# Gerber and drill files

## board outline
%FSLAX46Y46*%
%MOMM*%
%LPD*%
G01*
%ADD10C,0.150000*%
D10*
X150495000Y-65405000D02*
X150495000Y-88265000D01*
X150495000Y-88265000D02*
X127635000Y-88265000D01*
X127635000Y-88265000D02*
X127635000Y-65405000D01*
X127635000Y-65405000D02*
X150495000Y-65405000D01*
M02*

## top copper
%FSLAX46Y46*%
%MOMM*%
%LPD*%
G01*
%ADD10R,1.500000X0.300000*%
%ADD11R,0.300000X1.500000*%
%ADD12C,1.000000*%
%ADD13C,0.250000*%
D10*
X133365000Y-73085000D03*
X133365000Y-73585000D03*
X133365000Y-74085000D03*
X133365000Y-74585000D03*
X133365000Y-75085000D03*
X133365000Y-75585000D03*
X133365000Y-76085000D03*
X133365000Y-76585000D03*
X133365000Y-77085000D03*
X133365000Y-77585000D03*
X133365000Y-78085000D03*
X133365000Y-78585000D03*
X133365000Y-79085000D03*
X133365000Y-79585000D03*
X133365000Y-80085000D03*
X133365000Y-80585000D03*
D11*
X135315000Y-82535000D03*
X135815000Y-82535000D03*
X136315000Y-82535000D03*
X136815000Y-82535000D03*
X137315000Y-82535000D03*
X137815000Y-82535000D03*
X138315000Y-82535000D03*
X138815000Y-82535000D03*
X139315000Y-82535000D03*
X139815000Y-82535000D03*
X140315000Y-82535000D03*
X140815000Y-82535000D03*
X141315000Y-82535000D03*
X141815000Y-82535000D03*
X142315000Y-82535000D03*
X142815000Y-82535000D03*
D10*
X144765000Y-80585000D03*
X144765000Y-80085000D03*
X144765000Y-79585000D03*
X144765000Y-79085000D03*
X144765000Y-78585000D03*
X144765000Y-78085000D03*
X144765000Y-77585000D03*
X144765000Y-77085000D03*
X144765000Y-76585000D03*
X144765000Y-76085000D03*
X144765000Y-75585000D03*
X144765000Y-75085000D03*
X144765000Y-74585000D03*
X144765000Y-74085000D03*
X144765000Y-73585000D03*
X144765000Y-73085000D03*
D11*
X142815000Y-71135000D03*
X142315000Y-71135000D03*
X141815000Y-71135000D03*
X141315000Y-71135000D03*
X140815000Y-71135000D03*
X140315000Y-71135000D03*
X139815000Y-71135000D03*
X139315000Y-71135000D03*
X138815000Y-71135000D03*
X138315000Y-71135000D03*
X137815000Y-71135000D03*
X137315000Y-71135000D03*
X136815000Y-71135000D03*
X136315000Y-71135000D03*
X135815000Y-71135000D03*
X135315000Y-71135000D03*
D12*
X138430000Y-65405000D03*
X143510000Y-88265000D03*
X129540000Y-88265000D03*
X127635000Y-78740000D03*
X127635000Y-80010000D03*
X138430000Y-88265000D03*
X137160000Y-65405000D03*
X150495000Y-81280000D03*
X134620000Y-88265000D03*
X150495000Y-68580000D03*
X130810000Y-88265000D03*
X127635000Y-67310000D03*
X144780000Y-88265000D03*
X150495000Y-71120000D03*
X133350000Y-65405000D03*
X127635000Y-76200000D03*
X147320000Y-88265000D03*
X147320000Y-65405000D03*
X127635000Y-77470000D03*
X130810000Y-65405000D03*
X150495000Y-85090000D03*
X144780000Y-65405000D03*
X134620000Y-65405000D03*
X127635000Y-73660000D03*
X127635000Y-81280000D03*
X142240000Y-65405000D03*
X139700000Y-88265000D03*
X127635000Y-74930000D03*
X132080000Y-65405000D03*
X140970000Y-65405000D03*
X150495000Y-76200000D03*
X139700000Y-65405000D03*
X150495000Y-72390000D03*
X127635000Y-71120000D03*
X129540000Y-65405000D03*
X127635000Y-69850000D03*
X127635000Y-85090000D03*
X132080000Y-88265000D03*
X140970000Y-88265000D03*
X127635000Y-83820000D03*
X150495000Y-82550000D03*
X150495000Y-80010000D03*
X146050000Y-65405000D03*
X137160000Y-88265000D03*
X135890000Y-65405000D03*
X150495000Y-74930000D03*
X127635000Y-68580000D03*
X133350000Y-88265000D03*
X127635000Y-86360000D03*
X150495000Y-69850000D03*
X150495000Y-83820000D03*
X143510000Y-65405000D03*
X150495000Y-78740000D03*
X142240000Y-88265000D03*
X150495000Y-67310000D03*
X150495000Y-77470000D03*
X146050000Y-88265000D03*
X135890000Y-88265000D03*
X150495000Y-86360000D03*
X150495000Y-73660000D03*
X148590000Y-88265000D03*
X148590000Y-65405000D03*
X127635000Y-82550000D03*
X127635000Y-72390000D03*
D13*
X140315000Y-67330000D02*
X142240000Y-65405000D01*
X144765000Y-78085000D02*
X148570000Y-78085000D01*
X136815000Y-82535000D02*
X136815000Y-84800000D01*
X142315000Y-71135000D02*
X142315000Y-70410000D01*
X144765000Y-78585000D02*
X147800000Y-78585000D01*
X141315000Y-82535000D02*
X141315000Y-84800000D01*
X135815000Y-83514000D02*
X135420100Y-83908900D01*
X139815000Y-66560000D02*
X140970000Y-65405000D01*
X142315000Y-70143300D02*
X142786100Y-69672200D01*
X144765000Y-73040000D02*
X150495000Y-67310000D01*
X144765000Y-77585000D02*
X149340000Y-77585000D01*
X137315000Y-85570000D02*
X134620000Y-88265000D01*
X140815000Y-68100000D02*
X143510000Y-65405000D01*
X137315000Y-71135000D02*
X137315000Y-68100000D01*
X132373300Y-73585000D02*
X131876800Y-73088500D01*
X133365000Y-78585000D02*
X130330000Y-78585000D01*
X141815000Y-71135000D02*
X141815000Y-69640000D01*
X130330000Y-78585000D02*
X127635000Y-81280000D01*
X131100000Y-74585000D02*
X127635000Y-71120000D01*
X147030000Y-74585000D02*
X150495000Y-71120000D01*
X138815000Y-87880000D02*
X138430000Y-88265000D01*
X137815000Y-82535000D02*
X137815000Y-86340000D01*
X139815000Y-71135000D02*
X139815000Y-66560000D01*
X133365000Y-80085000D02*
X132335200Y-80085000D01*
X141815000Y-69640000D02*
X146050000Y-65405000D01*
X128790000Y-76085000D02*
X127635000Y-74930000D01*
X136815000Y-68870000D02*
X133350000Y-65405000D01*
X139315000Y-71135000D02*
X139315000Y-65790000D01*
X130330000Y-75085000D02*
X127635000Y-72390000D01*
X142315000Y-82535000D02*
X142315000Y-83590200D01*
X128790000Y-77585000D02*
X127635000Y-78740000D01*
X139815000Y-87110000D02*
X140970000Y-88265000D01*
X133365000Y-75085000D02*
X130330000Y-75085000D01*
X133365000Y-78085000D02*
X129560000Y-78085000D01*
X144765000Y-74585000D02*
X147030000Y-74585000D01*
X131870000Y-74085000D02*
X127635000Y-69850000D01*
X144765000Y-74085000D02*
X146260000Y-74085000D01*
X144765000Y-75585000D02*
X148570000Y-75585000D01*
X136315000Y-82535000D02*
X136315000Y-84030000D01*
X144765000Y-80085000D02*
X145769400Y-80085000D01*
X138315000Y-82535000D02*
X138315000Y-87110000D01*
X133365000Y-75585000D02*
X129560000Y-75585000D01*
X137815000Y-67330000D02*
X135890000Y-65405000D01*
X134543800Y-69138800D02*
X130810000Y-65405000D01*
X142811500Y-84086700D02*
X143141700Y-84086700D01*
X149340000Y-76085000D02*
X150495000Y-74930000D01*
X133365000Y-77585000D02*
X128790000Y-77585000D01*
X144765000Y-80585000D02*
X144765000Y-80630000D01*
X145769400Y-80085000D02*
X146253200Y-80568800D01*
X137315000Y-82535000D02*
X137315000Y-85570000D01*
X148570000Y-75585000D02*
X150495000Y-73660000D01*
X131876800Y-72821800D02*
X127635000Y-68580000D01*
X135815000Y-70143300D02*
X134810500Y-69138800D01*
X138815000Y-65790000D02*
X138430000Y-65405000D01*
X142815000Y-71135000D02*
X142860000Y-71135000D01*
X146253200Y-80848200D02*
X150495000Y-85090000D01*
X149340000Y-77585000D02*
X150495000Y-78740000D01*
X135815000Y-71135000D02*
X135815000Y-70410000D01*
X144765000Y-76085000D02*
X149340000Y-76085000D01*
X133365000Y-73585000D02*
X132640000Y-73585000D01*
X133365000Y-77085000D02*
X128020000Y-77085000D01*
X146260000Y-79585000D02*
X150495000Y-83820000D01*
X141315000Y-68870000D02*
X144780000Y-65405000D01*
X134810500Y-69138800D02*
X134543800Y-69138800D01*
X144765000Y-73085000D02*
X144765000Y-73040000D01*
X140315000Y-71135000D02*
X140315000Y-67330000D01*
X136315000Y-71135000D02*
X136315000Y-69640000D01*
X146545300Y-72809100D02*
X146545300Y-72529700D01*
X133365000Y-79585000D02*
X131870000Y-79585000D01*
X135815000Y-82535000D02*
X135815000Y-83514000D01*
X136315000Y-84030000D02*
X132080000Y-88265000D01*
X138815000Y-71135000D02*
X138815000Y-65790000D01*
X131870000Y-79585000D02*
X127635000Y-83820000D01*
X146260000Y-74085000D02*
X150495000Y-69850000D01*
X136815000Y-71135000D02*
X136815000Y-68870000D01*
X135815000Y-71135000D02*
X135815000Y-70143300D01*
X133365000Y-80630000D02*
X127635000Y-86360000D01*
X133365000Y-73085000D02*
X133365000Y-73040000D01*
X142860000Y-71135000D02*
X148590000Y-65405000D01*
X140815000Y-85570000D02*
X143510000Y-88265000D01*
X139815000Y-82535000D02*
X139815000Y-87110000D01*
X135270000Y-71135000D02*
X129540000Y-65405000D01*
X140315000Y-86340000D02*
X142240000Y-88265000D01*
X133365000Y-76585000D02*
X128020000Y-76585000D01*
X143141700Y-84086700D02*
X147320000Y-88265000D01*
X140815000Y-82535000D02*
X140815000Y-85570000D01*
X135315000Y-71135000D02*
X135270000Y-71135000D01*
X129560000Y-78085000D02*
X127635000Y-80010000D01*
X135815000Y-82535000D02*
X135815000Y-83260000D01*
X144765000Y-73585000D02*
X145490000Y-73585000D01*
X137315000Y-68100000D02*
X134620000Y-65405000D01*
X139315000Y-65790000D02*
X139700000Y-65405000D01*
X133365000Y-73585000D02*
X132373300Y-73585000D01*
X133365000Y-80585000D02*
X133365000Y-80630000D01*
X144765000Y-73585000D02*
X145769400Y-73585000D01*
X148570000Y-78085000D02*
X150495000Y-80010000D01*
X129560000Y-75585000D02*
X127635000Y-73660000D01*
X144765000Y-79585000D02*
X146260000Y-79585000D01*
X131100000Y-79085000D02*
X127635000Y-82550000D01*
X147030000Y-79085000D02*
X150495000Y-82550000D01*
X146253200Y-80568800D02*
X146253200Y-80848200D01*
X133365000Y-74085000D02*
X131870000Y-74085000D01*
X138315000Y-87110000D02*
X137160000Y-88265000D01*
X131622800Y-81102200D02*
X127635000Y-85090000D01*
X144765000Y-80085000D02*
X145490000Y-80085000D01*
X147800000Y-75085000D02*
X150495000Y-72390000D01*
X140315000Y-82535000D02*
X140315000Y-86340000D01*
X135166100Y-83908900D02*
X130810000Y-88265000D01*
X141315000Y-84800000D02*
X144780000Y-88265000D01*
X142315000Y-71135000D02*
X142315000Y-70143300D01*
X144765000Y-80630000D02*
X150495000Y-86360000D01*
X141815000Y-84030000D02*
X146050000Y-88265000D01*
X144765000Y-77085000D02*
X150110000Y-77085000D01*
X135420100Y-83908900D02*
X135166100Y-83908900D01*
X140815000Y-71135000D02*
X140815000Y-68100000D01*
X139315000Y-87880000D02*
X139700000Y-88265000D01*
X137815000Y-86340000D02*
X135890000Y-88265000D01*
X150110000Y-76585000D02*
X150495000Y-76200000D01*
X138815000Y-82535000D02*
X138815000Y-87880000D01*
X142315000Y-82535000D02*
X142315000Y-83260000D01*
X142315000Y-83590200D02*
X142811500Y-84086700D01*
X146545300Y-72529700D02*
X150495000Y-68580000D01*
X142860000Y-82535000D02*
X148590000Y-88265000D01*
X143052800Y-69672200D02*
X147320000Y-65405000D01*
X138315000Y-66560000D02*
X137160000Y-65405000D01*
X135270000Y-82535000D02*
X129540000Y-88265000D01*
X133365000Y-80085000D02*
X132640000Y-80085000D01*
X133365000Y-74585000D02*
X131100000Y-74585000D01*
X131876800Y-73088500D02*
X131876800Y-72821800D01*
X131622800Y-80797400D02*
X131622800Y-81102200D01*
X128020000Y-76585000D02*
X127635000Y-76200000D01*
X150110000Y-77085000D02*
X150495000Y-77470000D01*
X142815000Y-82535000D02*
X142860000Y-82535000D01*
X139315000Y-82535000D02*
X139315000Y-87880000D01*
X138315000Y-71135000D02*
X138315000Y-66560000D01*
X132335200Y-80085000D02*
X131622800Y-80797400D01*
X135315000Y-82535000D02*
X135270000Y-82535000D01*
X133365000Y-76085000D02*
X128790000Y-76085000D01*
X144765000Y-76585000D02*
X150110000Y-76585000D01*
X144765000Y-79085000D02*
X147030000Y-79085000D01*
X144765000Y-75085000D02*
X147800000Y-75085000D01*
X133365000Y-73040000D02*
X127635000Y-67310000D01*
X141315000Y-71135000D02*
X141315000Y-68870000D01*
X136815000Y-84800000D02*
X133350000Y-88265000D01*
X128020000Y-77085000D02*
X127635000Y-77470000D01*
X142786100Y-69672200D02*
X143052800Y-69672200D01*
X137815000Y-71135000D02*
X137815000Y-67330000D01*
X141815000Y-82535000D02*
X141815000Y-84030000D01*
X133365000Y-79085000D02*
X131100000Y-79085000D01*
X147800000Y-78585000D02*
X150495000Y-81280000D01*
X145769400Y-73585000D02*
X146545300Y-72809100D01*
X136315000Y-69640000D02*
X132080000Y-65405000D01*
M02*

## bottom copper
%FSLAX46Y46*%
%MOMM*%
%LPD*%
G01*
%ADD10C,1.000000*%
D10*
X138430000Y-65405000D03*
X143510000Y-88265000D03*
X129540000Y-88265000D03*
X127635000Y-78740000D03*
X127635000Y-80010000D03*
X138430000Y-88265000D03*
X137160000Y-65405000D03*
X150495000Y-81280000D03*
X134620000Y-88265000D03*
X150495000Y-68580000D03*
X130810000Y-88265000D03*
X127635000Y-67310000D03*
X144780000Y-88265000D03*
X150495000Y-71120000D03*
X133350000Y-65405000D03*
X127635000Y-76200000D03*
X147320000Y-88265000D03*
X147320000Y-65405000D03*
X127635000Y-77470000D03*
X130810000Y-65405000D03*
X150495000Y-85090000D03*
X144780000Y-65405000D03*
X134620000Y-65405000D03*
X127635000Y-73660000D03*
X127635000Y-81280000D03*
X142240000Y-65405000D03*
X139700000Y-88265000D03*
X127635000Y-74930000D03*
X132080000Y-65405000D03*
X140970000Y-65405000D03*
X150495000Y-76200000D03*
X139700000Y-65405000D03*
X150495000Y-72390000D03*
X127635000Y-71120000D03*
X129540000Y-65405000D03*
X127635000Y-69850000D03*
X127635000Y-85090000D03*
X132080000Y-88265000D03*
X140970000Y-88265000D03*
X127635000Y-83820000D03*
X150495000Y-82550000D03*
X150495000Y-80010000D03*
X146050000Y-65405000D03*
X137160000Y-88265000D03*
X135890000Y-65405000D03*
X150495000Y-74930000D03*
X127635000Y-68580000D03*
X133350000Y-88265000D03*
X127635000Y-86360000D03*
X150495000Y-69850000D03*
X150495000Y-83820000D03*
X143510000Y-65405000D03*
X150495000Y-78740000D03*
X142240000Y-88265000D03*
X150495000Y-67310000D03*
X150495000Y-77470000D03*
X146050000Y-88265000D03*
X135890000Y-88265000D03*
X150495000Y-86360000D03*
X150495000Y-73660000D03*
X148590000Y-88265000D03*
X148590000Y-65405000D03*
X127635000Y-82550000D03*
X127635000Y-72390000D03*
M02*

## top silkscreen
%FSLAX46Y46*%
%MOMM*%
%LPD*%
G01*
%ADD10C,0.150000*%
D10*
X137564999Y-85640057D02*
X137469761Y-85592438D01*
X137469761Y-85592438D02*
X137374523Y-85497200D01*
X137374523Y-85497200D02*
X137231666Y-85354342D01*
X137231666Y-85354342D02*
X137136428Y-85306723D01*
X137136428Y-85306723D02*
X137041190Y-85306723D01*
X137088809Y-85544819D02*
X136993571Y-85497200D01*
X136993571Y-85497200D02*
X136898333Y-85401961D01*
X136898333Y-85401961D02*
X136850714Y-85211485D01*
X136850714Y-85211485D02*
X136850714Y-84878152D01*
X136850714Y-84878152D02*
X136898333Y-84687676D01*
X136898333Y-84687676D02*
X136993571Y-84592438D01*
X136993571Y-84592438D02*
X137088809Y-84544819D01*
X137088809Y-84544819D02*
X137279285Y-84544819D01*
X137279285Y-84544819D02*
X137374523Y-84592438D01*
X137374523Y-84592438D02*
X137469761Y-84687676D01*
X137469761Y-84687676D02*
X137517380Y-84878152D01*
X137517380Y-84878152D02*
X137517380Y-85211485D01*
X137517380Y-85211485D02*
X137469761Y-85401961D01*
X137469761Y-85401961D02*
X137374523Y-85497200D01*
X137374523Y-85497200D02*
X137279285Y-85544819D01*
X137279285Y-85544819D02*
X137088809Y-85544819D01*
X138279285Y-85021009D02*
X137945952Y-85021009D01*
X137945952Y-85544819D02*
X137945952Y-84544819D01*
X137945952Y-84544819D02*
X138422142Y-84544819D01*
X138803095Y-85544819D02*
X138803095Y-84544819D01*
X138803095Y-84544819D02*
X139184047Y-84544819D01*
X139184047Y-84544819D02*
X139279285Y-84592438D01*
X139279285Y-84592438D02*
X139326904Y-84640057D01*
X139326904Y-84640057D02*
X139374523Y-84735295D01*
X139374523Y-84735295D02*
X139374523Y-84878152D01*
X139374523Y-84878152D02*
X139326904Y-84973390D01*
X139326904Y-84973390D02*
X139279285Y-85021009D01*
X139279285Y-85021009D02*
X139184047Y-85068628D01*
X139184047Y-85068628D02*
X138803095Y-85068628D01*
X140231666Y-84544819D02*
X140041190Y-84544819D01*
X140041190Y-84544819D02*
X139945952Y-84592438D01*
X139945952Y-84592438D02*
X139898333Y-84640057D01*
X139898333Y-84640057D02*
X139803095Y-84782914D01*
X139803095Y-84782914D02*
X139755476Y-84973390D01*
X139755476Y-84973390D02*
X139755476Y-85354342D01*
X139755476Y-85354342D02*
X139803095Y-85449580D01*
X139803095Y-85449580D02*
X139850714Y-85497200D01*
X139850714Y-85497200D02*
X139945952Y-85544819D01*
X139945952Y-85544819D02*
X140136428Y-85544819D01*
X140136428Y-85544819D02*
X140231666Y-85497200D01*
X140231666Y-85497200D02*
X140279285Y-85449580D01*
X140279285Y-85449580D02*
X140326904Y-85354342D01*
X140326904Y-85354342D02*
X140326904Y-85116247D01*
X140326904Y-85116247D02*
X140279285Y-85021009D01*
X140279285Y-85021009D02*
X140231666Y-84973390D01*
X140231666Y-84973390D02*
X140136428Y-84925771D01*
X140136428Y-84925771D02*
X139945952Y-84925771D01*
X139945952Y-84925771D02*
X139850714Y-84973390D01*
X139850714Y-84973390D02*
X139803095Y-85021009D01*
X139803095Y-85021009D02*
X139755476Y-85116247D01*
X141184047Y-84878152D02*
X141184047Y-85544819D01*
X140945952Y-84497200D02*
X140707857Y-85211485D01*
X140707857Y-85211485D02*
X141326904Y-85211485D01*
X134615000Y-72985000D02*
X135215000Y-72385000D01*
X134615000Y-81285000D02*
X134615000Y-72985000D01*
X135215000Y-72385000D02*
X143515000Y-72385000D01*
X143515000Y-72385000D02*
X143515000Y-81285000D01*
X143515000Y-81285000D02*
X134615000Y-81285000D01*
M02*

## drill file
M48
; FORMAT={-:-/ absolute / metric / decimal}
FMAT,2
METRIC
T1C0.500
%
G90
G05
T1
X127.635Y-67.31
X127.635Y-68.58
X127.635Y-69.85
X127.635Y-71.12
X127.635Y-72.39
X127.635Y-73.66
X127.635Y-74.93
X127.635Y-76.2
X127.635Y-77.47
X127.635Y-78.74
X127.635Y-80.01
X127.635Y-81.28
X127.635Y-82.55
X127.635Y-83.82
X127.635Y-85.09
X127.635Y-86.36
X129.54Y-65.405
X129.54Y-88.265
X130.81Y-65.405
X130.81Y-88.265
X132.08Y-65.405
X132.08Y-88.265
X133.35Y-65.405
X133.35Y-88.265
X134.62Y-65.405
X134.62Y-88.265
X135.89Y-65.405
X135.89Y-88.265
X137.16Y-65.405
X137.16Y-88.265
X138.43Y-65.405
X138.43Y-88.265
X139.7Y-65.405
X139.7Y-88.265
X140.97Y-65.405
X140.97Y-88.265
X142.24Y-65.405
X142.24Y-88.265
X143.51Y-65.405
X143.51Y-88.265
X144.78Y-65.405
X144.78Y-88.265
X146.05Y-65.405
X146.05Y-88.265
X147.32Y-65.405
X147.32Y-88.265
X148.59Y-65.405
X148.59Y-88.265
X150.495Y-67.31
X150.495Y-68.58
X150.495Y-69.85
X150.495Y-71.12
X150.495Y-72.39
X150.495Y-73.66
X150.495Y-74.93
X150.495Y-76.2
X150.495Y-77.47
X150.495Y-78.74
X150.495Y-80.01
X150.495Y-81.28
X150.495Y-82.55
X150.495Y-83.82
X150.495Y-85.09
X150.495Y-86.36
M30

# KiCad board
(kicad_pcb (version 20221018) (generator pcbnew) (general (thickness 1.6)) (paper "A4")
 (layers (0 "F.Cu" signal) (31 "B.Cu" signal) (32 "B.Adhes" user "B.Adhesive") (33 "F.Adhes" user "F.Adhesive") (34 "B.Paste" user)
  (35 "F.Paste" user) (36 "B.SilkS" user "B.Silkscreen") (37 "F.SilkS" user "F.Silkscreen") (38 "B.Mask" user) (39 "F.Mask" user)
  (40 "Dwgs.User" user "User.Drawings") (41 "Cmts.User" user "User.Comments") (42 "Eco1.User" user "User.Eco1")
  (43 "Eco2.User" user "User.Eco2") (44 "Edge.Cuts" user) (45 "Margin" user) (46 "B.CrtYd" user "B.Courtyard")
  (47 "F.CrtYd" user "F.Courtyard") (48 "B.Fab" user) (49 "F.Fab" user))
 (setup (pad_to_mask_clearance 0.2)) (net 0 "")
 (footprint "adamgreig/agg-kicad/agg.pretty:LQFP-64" (layer "F.Cu") (at 139.065 76.835)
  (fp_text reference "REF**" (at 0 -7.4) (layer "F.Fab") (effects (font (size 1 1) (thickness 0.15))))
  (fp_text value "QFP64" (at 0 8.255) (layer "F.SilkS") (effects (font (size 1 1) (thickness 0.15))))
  (fp_line (start -4.45 -3.85) (end -3.85 -4.45) (stroke (width 0.15) (type solid)) (layer "F.SilkS"))
  (fp_line (start -4.45 4.45) (end -4.45 -3.85) (stroke (width 0.15) (type solid)) (layer "F.SilkS"))
  (fp_line (start -3.85 -4.45) (end 4.45 -4.45) (stroke (width 0.15) (type solid)) (layer "F.SilkS"))
  (fp_line (start 4.45 -4.45) (end 4.45 4.45) (stroke (width 0.15) (type solid)) (layer "F.SilkS"))
  (fp_line (start 4.45 4.45) (end -4.45 4.45) (stroke (width 0.15) (type solid)) (layer "F.SilkS"))
  (pad "1" smd rect (at -5.7 -3.75) (size 1.5 0.3) (layers "F.Cu" "F.Paste" "F.Mask"))
  (pad "2" smd rect (at -5.7 -3.25) (size 1.5 0.3) (layers "F.Cu" "F.Paste" "F.Mask"))
  (pad "3" smd rect (at -5.7 -2.75) (size 1.5 0.3) (layers "F.Cu" "F.Paste" "F.Mask"))
  (pad "4" smd rect (at -5.7 -2.25) (size 1.5 0.3) (layers "F.Cu" "F.Paste" "F.Mask"))
  (pad "5" smd rect (at -5.7 -1.75) (size 1.5 0.3) (layers "F.Cu" "F.Paste" "F.Mask"))
  (pad "6" smd rect (at -5.7 -1.25) (size 1.5 0.3) (layers "F.Cu" "F.Paste" "F.Mask"))
  (pad "7" smd rect (at -5.7 -0.75) (size 1.5 0.3) (layers "F.Cu" "F.Paste" "F.Mask"))
  (pad "8" smd rect (at -5.7 -0.25) (size 1.5 0.3) (layers "F.Cu" "F.Paste" "F.Mask"))
  (pad "9" smd rect (at -5.7 0.25) (size 1.5 0.3) (layers "F.Cu" "F.Paste" "F.Mask"))
  (pad "10" smd rect (at -5.7 0.75) (size 1.5 0.3) (layers "F.Cu" "F.Paste" "F.Mask"))
  (pad "11" smd rect (at -5.7 1.25) (size 1.5 0.3) (layers "F.Cu" "F.Paste" "F.Mask"))
  (pad "12" smd rect (at -5.7 1.75) (size 1.5 0.3) (layers "F.Cu" "F.Paste" "F.Mask"))
  (pad "13" smd rect (at -5.7 2.25) (size 1.5 0.3) (layers "F.Cu" "F.Paste" "F.Mask"))
  (pad "14" smd rect (at -5.7 2.75) (size 1.5 0.3) (layers "F.Cu" "F.Paste" "F.Mask"))
  (pad "15" smd rect (at -5.7 3.25) (size 1.5 0.3) (layers "F.Cu" "F.Paste" "F.Mask"))
  (pad "16" smd rect (at -5.7 3.75) (size 1.5 0.3) (layers "F.Cu" "F.Paste" "F.Mask"))
  (pad "17" smd rect (at -3.75 5.7) (size 0.3 1.5) (layers "F.Cu" "F.Paste" "F.Mask"))
  (pad "18" smd rect (at -3.25 5.7) (size 0.3 1.5) (layers "F.Cu" "F.Paste" "F.Mask"))
  (pad "19" smd rect (at -2.75 5.7) (size 0.3 1.5) (layers "F.Cu" "F.Paste" "F.Mask"))
  (pad "20" smd rect (at -2.25 5.7) (size 0.3 1.5) (layers "F.Cu" "F.Paste" "F.Mask"))
  (pad "21" smd rect (at -1.75 5.7) (size 0.3 1.5) (layers "F.Cu" "F.Paste" "F.Mask"))
  (pad "22" smd rect (at -1.25 5.7) (size 0.3 1.5) (layers "F.Cu" "F.Paste" "F.Mask"))
  (pad "23" smd rect (at -0.75 5.7) (size 0.3 1.5) (layers "F.Cu" "F.Paste" "F.Mask"))
  (pad "24" smd rect (at -0.25 5.7) (size 0.3 1.5) (layers "F.Cu" "F.Paste" "F.Mask"))
  (pad "25" smd rect (at 0.25 5.7) (size 0.3 1.5) (layers "F.Cu" "F.Paste" "F.Mask"))
  (pad "26" smd rect (at 0.75 5.7) (size 0.3 1.5) (layers "F.Cu" "F.Paste" "F.Mask"))
  (pad "27" smd rect (at 1.25 5.7) (size 0.3 1.5) (layers "F.Cu" "F.Paste" "F.Mask"))
  (pad "28" smd rect (at 1.75 5.7) (size 0.3 1.5) (layers "F.Cu" "F.Paste" "F.Mask"))
  (pad "29" smd rect (at 2.25 5.7) (size 0.3 1.5) (layers "F.Cu" "F.Paste" "F.Mask"))
  (pad "30" smd rect (at 2.75 5.7) (size 0.3 1.5) (layers "F.Cu" "F.Paste" "F.Mask"))
  (pad "31" smd rect (at 3.25 5.7) (size 0.3 1.5) (layers "F.Cu" "F.Paste" "F.Mask"))
  (pad "32" smd rect (at 3.75 5.7) (size 0.3 1.5) (layers "F.Cu" "F.Paste" "F.Mask"))
  (pad "33" smd rect (at 5.7 3.75) (size 1.5 0.3) (layers "F.Cu" "F.Paste" "F.Mask"))
  (pad "34" smd rect (at 5.7 3.25) (size 1.5 0.3) (layers "F.Cu" "F.Paste" "F.Mask"))
  (pad "35" smd rect (at 5.7 2.75) (size 1.5 0.3) (layers "F.Cu" "F.Paste" "F.Mask"))
  (pad "36" smd rect (at 5.7 2.25) (size 1.5 0.3) (layers "F.Cu" "F.Paste" "F.Mask"))
  (pad "37" smd rect (at 5.7 1.75) (size 1.5 0.3) (layers "F.Cu" "F.Paste" "F.Mask"))
  (pad "38" smd rect (at 5.7 1.25) (size 1.5 0.3) (layers "F.Cu" "F.Paste" "F.Mask"))
  (pad "39" smd rect (at 5.7 0.75) (size 1.5 0.3) (layers "F.Cu" "F.Paste" "F.Mask"))
  (pad "40" smd rect (at 5.7 0.25) (size 1.5 0.3) (layers "F.Cu" "F.Paste" "F.Mask"))
  (pad "41" smd rect (at 5.7 -0.25) (size 1.5 0.3) (layers "F.Cu" "F.Paste" "F.Mask"))
  (pad "42" smd rect (at 5.7 -0.75) (size 1.5 0.3) (layers "F.Cu" "F.Paste" "F.Mask"))
  (pad "43" smd rect (at 5.7 -1.25) (size 1.5 0.3) (layers "F.Cu" "F.Paste" "F.Mask"))
  (pad "44" smd rect (at 5.7 -1.75) (size 1.5 0.3) (layers "F.Cu" "F.Paste" "F.Mask"))
  (pad "45" smd rect (at 5.7 -2.25) (size 1.5 0.3) (layers "F.Cu" "F.Paste" "F.Mask"))
  (pad "46" smd rect (at 5.7 -2.75) (size 1.5 0.3) (layers "F.Cu" "F.Paste" "F.Mask"))
  (pad "47" smd rect (at 5.7 -3.25) (size 1.5 0.3) (layers "F.Cu" "F.Paste" "F.Mask"))
  (pad "48" smd rect (at 5.7 -3.75) (size 1.5 0.3) (layers "F.Cu" "F.Paste" "F.Mask"))
  (pad "49" smd rect (at 3.75 -5.7) (size 0.3 1.5) (layers "F.Cu" "F.Paste" "F.Mask"))
  (pad "50" smd rect (at 3.25 -5.7) (size 0.3 1.5) (layers "F.Cu" "F.Paste" "F.Mask"))
  (pad "51" smd rect (at 2.75 -5.7) (size 0.3 1.5) (layers "F.Cu" "F.Paste" "F.Mask"))
  (pad "52" smd rect (at 2.25 -5.7) (size 0.3 1.5) (layers "F.Cu" "F.Paste" "F.Mask"))
  (pad "53" smd rect (at 1.75 -5.7) (size 0.3 1.5) (layers "F.Cu" "F.Paste" "F.Mask"))
  (pad "54" smd rect (at 1.25 -5.7) (size 0.3 1.5) (layers "F.Cu" "F.Paste" "F.Mask"))
  (pad "55" smd rect (at 0.75 -5.7) (size 0.3 1.5) (layers "F.Cu" "F.Paste" "F.Mask"))
  (pad "56" smd rect (at 0.25 -5.7) (size 0.3 1.5) (layers "F.Cu" "F.Paste" "F.Mask"))
  (pad "57" smd rect (at -0.25 -5.7) (size 0.3 1.5) (layers "F.Cu" "F.Paste" "F.Mask"))
  (pad "58" smd rect (at -0.75 -5.7) (size 0.3 1.5) (layers "F.Cu" "F.Paste" "F.Mask"))
  (pad "59" smd rect (at -1.25 -5.7) (size 0.3 1.5) (layers "F.Cu" "F.Paste" "F.Mask"))
  (pad "60" smd rect (at -1.75 -5.7) (size 0.3 1.5) (layers "F.Cu" "F.Paste" "F.Mask"))
  (pad "61" smd rect (at -2.25 -5.7) (size 0.3 1.5) (layers "F.Cu" "F.Paste" "F.Mask"))
  (pad "62" smd rect (at -2.75 -5.7) (size 0.3 1.5) (layers "F.Cu" "F.Paste" "F.Mask"))
  (pad "63" smd rect (at -3.25 -5.7) (size 0.3 1.5) (layers "F.Cu" "F.Paste" "F.Mask"))
  (pad "64" smd rect (at -3.75 -5.7) (size 0.3 1.5) (layers "F.Cu" "F.Paste" "F.Mask")))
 (gr_line (start 150.495 65.405) (end 150.495 88.265) (stroke (width 0.15) (type solid)) (layer "Edge.Cuts"))
 (gr_line (start 150.495 88.265) (end 127.635 88.265) (stroke (width 0.15) (type solid)) (layer "Edge.Cuts"))
 (gr_line (start 127.635 88.265) (end 127.635 65.405) (stroke (width 0.15) (type solid)) (layer "Edge.Cuts"))
 (gr_line (start 127.635 65.405) (end 150.495 65.405) (stroke (width 0.15) (type solid)) (layer "Edge.Cuts"))
 (segment (start 140.315 67.33) (end 142.24 65.405) (width 0.25) (layer "F.Cu") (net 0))
 (segment (start 144.765 78.085) (end 148.57 78.085) (width 0.25) (layer "F.Cu") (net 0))
 (segment (start 136.815 82.535) (end 136.815 84.8) (width 0.25) (layer "F.Cu") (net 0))
 (segment (start 142.315 71.135) (end 142.315 70.41) (width 0.25) (layer "F.Cu") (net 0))
 (segment (start 144.765 78.585) (end 147.8 78.585) (width 0.25) (layer "F.Cu") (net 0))
 (segment (start 141.315 82.535) (end 141.315 84.8) (width 0.25) (layer "F.Cu") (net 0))
 (segment (start 135.815 83.514) (end 135.4201 83.9089) (width 0.25) (layer "F.Cu") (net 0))
 (segment (start 139.815 66.56) (end 140.97 65.405) (width 0.25) (layer "F.Cu") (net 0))
 (segment (start 142.315 70.1433) (end 142.7861 69.6722) (width 0.25) (layer "F.Cu") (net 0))
 (segment (start 144.765 73.04) (end 150.495 67.31) (width 0.25) (layer "F.Cu") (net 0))
 (segment (start 144.765 77.585) (end 149.34 77.585) (width 0.25) (layer "F.Cu") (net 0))
 (segment (start 137.315 85.57) (end 134.62 88.265) (width 0.25) (layer "F.Cu") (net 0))
 (segment (start 140.815 68.1) (end 143.51 65.405) (width 0.25) (layer "F.Cu") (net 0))
 (segment (start 137.315 71.135) (end 137.315 68.1) (width 0.25) (layer "F.Cu") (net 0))
 (segment (start 132.3733 73.585) (end 131.8768 73.0885) (width 0.25) (layer "F.Cu") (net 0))
 (segment (start 133.365 78.585) (end 130.33 78.585) (width 0.25) (layer "F.Cu") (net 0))
 (segment (start 141.815 71.135) (end 141.815 69.64) (width 0.25) (layer "F.Cu") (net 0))
 (segment (start 130.33 78.585) (end 127.635 81.28) (width 0.25) (layer "F.Cu") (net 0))
 (segment (start 131.1 74.585) (end 127.635 71.12) (width 0.25) (layer "F.Cu") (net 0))
 (segment (start 147.03 74.585) (end 150.495 71.12) (width 0.25) (layer "F.Cu") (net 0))
 (segment (start 138.815 87.88) (end 138.43 88.265) (width 0.25) (layer "F.Cu") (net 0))
 (segment (start 137.815 82.535) (end 137.815 86.34) (width 0.25) (layer "F.Cu") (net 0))
 (segment (start 139.815 71.135) (end 139.815 66.56) (width 0.25) (layer "F.Cu") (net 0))
 (segment (start 133.365 80.085) (end 132.3352 80.085) (width 0.25) (layer "F.Cu") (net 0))
 (segment (start 141.815 69.64) (end 146.05 65.405) (width 0.25) (layer "F.Cu") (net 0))
 (segment (start 128.79 76.085) (end 127.635 74.93) (width 0.25) (layer "F.Cu") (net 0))
 (segment (start 136.815 68.87) (end 133.35 65.405) (width 0.25) (layer "F.Cu") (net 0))
 (segment (start 139.315 71.135) (end 139.315 65.79) (width 0.25) (layer "F.Cu") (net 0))
 (segment (start 130.33 75.085) (end 127.635 72.39) (width 0.25) (layer "F.Cu") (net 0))
 (segment (start 142.315 82.535) (end 142.315 83.5902) (width 0.25) (layer "F.Cu") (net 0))
 (segment (start 128.79 77.585) (end 127.635 78.74) (width 0.25) (layer "F.Cu") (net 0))
 (segment (start 139.815 87.11) (end 140.97 88.265) (width 0.25) (layer "F.Cu") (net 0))
 (segment (start 133.365 75.085) (end 130.33 75.085) (width 0.25) (layer "F.Cu") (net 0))
 (segment (start 133.365 78.085) (end 129.56 78.085) (width 0.25) (layer "F.Cu") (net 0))
 (segment (start 144.765 74.585) (end 147.03 74.585) (width 0.25) (layer "F.Cu") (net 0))
 (segment (start 131.87 74.085) (end 127.635 69.85) (width 0.25) (layer "F.Cu") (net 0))
 (segment (start 144.765 74.085) (end 146.26 74.085) (width 0.25) (layer "F.Cu") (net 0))
 (segment (start 144.765 75.585) (end 148.57 75.585) (width 0.25) (layer "F.Cu") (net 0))
 (segment (start 136.315 82.535) (end 136.315 84.03) (width 0.25) (layer "F.Cu") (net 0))
 (segment (start 144.765 80.085) (end 145.7694 80.085) (width 0.25) (layer "F.Cu") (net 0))
 (segment (start 138.315 82.535) (end 138.315 87.11) (width 0.25) (layer "F.Cu") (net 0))
 (segment (start 133.365 75.585) (end 129.56 75.585) (width 0.25) (layer "F.Cu") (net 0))
 (segment (start 137.815 67.33) (end 135.89 65.405) (width 0.25) (layer "F.Cu") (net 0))
 (segment (start 134.5438 69.1388) (end 130.81 65.405) (width 0.25) (layer "F.Cu") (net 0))
 (segment (start 142.8115 84.0867) (end 143.1417 84.0867) (width 0.25) (layer "F.Cu") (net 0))
 (segment (start 149.34 76.085) (end 150.495 74.93) (width 0.25) (layer "F.Cu") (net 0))
 (segment (start 133.365 77.585) (end 128.79 77.585) (width 0.25) (layer "F.Cu") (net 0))
 (segment (start 144.765 80.585) (end 144.765 80.63) (width 0.25) (layer "F.Cu") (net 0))
 (segment (start 145.7694 80.085) (end 146.2532 80.5688) (width 0.25) (layer "F.Cu") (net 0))
 (segment (start 137.315 82.535) (end 137.315 85.57) (width 0.25) (layer "F.Cu") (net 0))
 (segment (start 148.57 75.585) (end 150.495 73.66) (width 0.25) (layer "F.Cu") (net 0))
 (segment (start 131.8768 72.8218) (end 127.635 68.58) (width 0.25) (layer "F.Cu") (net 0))
 (segment (start 135.815 70.1433) (end 134.8105 69.1388) (width 0.25) (layer "F.Cu") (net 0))
 (segment (start 138.815 65.79) (end 138.43 65.405) (width 0.25) (layer "F.Cu") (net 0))
 (segment (start 142.815 71.135) (end 142.86 71.135) (width 0.25) (layer "F.Cu") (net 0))
 (segment (start 146.2532 80.8482) (end 150.495 85.09) (width 0.25) (layer "F.Cu") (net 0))
 (segment (start 149.34 77.585) (end 150.495 78.74) (width 0.25) (layer "F.Cu") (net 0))
 (segment (start 135.815 71.135) (end 135.815 70.41) (width 0.25) (layer "F.Cu") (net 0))
 (segment (start 144.765 76.085) (end 149.34 76.085) (width 0.25) (layer "F.Cu") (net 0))
 (segment (start 133.365 73.585) (end 132.64 73.585) (width 0.25) (layer "F.Cu") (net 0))
 (segment (start 133.365 77.085) (end 128.02 77.085) (width 0.25) (layer "F.Cu") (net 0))
 (segment (start 146.26 79.585) (end 150.495 83.82) (width 0.25) (layer "F.Cu") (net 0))
 (segment (start 141.315 68.87) (end 144.78 65.405) (width 0.25) (layer "F.Cu") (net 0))
 (segment (start 134.8105 69.1388) (end 134.5438 69.1388) (width 0.25) (layer "F.Cu") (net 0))
 (segment (start 144.765 73.085) (end 144.765 73.04) (width 0.25) (layer "F.Cu") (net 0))
 (segment (start 140.315 71.135) (end 140.315 67.33) (width 0.25) (layer "F.Cu") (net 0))
 (segment (start 136.315 71.135) (end 136.315 69.64) (width 0.25) (layer "F.Cu") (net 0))
 (segment (start 146.5453 72.8091) (end 146.5453 72.5297) (width 0.25) (layer "F.Cu") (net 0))
 (segment (start 133.365 79.585) (end 131.87 79.585) (width 0.25) (layer "F.Cu") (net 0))
 (segment (start 135.815 82.535) (end 135.815 83.514) (width 0.25) (layer "F.Cu") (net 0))
 (segment (start 136.315 84.03) (end 132.08 88.265) (width 0.25) (layer "F.Cu") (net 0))
 (segment (start 138.815 71.135) (end 138.815 65.79) (width 0.25) (layer "F.Cu") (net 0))
 (segment (start 131.87 79.585) (end 127.635 83.82) (width 0.25) (layer "F.Cu") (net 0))
 (segment (start 146.26 74.085) (end 150.495 69.85) (width 0.25) (layer "F.Cu") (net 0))
 (segment (start 136.815 71.135) (end 136.815 68.87) (width 0.25) (layer "F.Cu") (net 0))
 (segment (start 135.815 71.135) (end 135.815 70.1433) (width 0.25) (layer "F.Cu") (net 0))
 (segment (start 133.365 80.63) (end 127.635 86.36) (width 0.25) (layer "F.Cu") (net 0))
 (segment (start 133.365 73.085) (end 133.365 73.04) (width 0.25) (layer "F.Cu") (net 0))
 (segment (start 142.86 71.135) (end 148.59 65.405) (width 0.25) (layer "F.Cu") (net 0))
 (segment (start 140.815 85.57) (end 143.51 88.265) (width 0.25) (layer "F.Cu") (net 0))
 (segment (start 139.815 82.535) (end 139.815 87.11) (width 0.25) (layer "F.Cu") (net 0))
 (segment (start 135.27 71.135) (end 129.54 65.405) (width 0.25) (layer "F.Cu") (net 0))
 (segment (start 140.315 86.34) (end 142.24 88.265) (width 0.25) (layer "F.Cu") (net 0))
 (segment (start 133.365 76.585) (end 128.02 76.585) (width 0.25) (layer "F.Cu") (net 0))
 (segment (start 143.1417 84.0867) (end 147.32 88.265) (width 0.25) (layer "F.Cu") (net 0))
 (segment (start 140.815 82.535) (end 140.815 85.57) (width 0.25) (layer "F.Cu") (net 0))
 (segment (start 135.315 71.135) (end 135.27 71.135) (width 0.25) (layer "F.Cu") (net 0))
 (segment (start 129.56 78.085) (end 127.635 80.01) (width 0.25) (layer "F.Cu") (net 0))
 (segment (start 135.815 82.535) (end 135.815 83.26) (width 0.25) (layer "F.Cu") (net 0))
 (segment (start 144.765 73.585) (end 145.49 73.585) (width 0.25) (layer "F.Cu") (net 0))
 (segment (start 137.315 68.1) (end 134.62 65.405) (width 0.25) (layer "F.Cu") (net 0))
 (segment (start 139.315 65.79) (end 139.7 65.405) (width 0.25) (layer "F.Cu") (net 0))
 (segment (start 133.365 73.585) (end 132.3733 73.585) (width 0.25) (layer "F.Cu") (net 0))
 (segment (start 133.365 80.585) (end 133.365 80.63) (width 0.25) (layer "F.Cu") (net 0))
 (segment (start 144.765 73.585) (end 145.7694 73.585) (width 0.25) (layer "F.Cu") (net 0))
 (segment (start 148.57 78.085) (end 150.495 80.01) (width 0.25) (layer "F.Cu") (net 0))
 (segment (start 129.56 75.585) (end 127.635 73.66) (width 0.25) (layer "F.Cu") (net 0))
 (segment (start 144.765 79.585) (end 146.26 79.585) (width 0.25) (layer "F.Cu") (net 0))
 (segment (start 131.1 79.085) (end 127.635 82.55) (width 0.25) (layer "F.Cu") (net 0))
 (segment (start 147.03 79.085) (end 150.495 82.55) (width 0.25) (layer "F.Cu") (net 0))
 (segment (start 146.2532 80.5688) (end 146.2532 80.8482) (width 0.25) (layer "F.Cu") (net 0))
 (segment (start 133.365 74.085) (end 131.87 74.085) (width 0.25) (layer "F.Cu") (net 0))
 (segment (start 138.315 87.11) (end 137.16 88.265) (width 0.25) (layer "F.Cu") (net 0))
 (segment (start 131.6228 81.1022) (end 127.635 85.09) (width 0.25) (layer "F.Cu") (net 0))
 (segment (start 144.765 80.085) (end 145.49 80.085) (width 0.25) (layer "F.Cu") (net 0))
 (segment (start 147.8 75.085) (end 150.495 72.39) (width 0.25) (layer "F.Cu") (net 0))
 (segment (start 140.315 82.535) (end 140.315 86.34) (width 0.25) (layer "F.Cu") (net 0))
 (segment (start 135.1661 83.9089) (end 130.81 88.265) (width 0.25) (layer "F.Cu") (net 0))
 (segment (start 141.315 84.8) (end 144.78 88.265) (width 0.25) (layer "F.Cu") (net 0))
 (segment (start 142.315 71.135) (end 142.315 70.1433) (width 0.25) (layer "F.Cu") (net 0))
 (segment (start 144.765 80.63) (end 150.495 86.36) (width 0.25) (layer "F.Cu") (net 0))
 (segment (start 141.815 84.03) (end 146.05 88.265) (width 0.25) (layer "F.Cu") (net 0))
 (segment (start 144.765 77.085) (end 150.11 77.085) (width 0.25) (layer "F.Cu") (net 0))
 (segment (start 135.4201 83.9089) (end 135.1661 83.9089) (width 0.25) (layer "F.Cu") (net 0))
 (segment (start 140.815 71.135) (end 140.815 68.1) (width 0.25) (layer "F.Cu") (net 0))
 (segment (start 139.315 87.88) (end 139.7 88.265) (width 0.25) (layer "F.Cu") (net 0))
 (segment (start 137.815 86.34) (end 135.89 88.265) (width 0.25) (layer "F.Cu") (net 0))
 (segment (start 150.11 76.585) (end 150.495 76.2) (width 0.25) (layer "F.Cu") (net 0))
 (segment (start 138.815 82.535) (end 138.815 87.88) (width 0.25) (layer "F.Cu") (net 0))
 (segment (start 142.315 82.535) (end 142.315 83.26) (width 0.25) (layer "F.Cu") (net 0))
 (segment (start 142.315 83.5902) (end 142.8115 84.0867) (width 0.25) (layer "F.Cu") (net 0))
 (segment (start 146.5453 72.5297) (end 150.495 68.58) (width 0.25) (layer "F.Cu") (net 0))
 (segment (start 142.86 82.535) (end 148.59 88.265) (width 0.25) (layer "F.Cu") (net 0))
 (segment (start 143.0528 69.6722) (end 147.32 65.405) (width 0.25) (layer "F.Cu") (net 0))
 (segment (start 138.315 66.56) (end 137.16 65.405) (width 0.25) (layer "F.Cu") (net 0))
 (segment (start 135.27 82.535) (end 129.54 88.265) (width 0.25) (layer "F.Cu") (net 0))
 (segment (start 133.365 80.085) (end 132.64 80.085) (width 0.25) (layer "F.Cu") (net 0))
 (segment (start 133.365 74.585) (end 131.1 74.585) (width 0.25) (layer "F.Cu") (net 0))
 (segment (start 131.8768 73.0885) (end 131.8768 72.8218) (width 0.25) (layer "F.Cu") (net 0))
 (segment (start 131.6228 80.7974) (end 131.6228 81.1022) (width 0.25) (layer "F.Cu") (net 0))
 (segment (start 128.02 76.585) (end 127.635 76.2) (width 0.25) (layer "F.Cu") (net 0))
 (segment (start 150.11 77.085) (end 150.495 77.47) (width 0.25) (layer "F.Cu") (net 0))
 (segment (start 142.815 82.535) (end 142.86 82.535) (width 0.25) (layer "F.Cu") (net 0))
 (segment (start 139.315 82.535) (end 139.315 87.88) (width 0.25) (layer "F.Cu") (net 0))
 (segment (start 138.315 71.135) (end 138.315 66.56) (width 0.25) (layer "F.Cu") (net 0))
 (segment (start 132.3352 80.085) (end 131.6228 80.7974) (width 0.25) (layer "F.Cu") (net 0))
 (segment (start 135.315 82.535) (end 135.27 82.535) (width 0.25) (layer "F.Cu") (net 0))
 (segment (start 133.365 76.085) (end 128.79 76.085) (width 0.25) (layer "F.Cu") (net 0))
 (segment (start 144.765 76.585) (end 150.11 76.585) (width 0.25) (layer "F.Cu") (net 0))
 (segment (start 144.765 79.085) (end 147.03 79.085) (width 0.25) (layer "F.Cu") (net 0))
 (segment (start 144.765 75.085) (end 147.8 75.085) (width 0.25) (layer "F.Cu") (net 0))
 (segment (start 133.365 73.04) (end 127.635 67.31) (width 0.25) (layer "F.Cu") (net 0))
 (segment (start 141.315 71.135) (end 141.315 68.87) (width 0.25) (layer "F.Cu") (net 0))
 (segment (start 136.815 84.8) (end 133.35 88.265) (width 0.25) (layer "F.Cu") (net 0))
 (segment (start 128.02 77.085) (end 127.635 77.47) (width 0.25) (layer "F.Cu") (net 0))
 (segment (start 142.7861 69.6722) (end 143.0528 69.6722) (width 0.25) (layer "F.Cu") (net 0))
 (segment (start 137.815 71.135) (end 137.815 67.33) (width 0.25) (layer "F.Cu") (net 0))
 (segment (start 141.815 82.535) (end 141.815 84.03) (width 0.25) (layer "F.Cu") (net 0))
 (segment (start 133.365 79.085) (end 131.1 79.085) (width 0.25) (layer "F.Cu") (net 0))
 (segment (start 147.8 78.585) (end 150.495 81.28) (width 0.25) (layer "F.Cu") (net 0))
 (segment (start 145.7694 73.585) (end 146.5453 72.8091) (width 0.25) (layer "F.Cu") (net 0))
 (segment (start 136.315 69.64) (end 132.08 65.405) (width 0.25) (layer "F.Cu") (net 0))
 (via (at 138.43 65.405) (size 1) (drill 0.5) (layers "F.Cu" "B.Cu") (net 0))
 (via (at 143.51 88.265) (size 1) (drill 0.5) (layers "F.Cu" "B.Cu") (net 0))
 (via (at 129.54 88.265) (size 1) (drill 0.5) (layers "F.Cu" "B.Cu") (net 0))
 (via (at 127.635 78.74) (size 1) (drill 0.5) (layers "F.Cu" "B.Cu") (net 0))
 (via (at 127.635 80.01) (size 1) (drill 0.5) (layers "F.Cu" "B.Cu") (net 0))
 (via (at 138.43 88.265) (size 1) (drill 0.5) (layers "F.Cu" "B.Cu") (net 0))
 (via (at 137.16 65.405) (size 1) (drill 0.5) (layers "F.Cu" "B.Cu") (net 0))
 (via (at 150.495 81.28) (size 1) (drill 0.5) (layers "F.Cu" "B.Cu") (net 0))
 (via (at 134.62 88.265) (size 1) (drill 0.5) (layers "F.Cu" "B.Cu") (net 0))
 (via (at 150.495 68.58) (size 1) (drill 0.5) (layers "F.Cu" "B.Cu") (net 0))
 (via (at 130.81 88.265) (size 1) (drill 0.5) (layers "F.Cu" "B.Cu") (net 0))
 (via (at 127.635 67.31) (size 1) (drill 0.5) (layers "F.Cu" "B.Cu") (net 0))
 (via (at 144.78 88.265) (size 1) (drill 0.5) (layers "F.Cu" "B.Cu") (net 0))
 (via (at 150.495 71.12) (size 1) (drill 0.5) (layers "F.Cu" "B.Cu") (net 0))
 (via (at 133.35 65.405) (size 1) (drill 0.5) (layers "F.Cu" "B.Cu") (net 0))
 (via (at 127.635 76.2) (size 1) (drill 0.5) (layers "F.Cu" "B.Cu") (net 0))
 (via (at 147.32 88.265) (size 1) (drill 0.5) (layers "F.Cu" "B.Cu") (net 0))
 (via (at 147.32 65.405) (size 1) (drill 0.5) (layers "F.Cu" "B.Cu") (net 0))
 (via (at 127.635 77.47) (size 1) (drill 0.5) (layers "F.Cu" "B.Cu") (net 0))
 (via (at 130.81 65.405) (size 1) (drill 0.5) (layers "F.Cu" "B.Cu") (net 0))
 (via (at 150.495 85.09) (size 1) (drill 0.5) (layers "F.Cu" "B.Cu") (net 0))
 (via (at 144.78 65.405) (size 1) (drill 0.5) (layers "F.Cu" "B.Cu") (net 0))
 (via (at 134.62 65.405) (size 1) (drill 0.5) (layers "F.Cu" "B.Cu") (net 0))
 (via (at 127.635 73.66) (size 1) (drill 0.5) (layers "F.Cu" "B.Cu") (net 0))
 (via (at 127.635 81.28) (size 1) (drill 0.5) (layers "F.Cu" "B.Cu") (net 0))
 (via (at 142.24 65.405) (size 1) (drill 0.5) (layers "F.Cu" "B.Cu") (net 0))
 (via (at 139.7 88.265) (size 1) (drill 0.5) (layers "F.Cu" "B.Cu") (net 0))
 (via (at 127.635 74.93) (size 1) (drill 0.5) (layers "F.Cu" "B.Cu") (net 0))
 (via (at 132.08 65.405) (size 1) (drill 0.5) (layers "F.Cu" "B.Cu") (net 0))
 (via (at 140.97 65.405) (size 1) (drill 0.5) (layers "F.Cu" "B.Cu") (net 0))
 (via (at 150.495 76.2) (size 1) (drill 0.5) (layers "F.Cu" "B.Cu") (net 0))
 (via (at 139.7 65.405) (size 1) (drill 0.5) (layers "F.Cu" "B.Cu") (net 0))
 (via (at 150.495 72.39) (size 1) (drill 0.5) (layers "F.Cu" "B.Cu") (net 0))
 (via (at 127.635 71.12) (size 1) (drill 0.5) (layers "F.Cu" "B.Cu") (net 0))
 (via (at 129.54 65.405) (size 1) (drill 0.5) (layers "F.Cu" "B.Cu") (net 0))
 (via (at 127.635 69.85) (size 1) (drill 0.5) (layers "F.Cu" "B.Cu") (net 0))
 (via (at 127.635 85.09) (size 1) (drill 0.5) (layers "F.Cu" "B.Cu") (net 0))
 (via (at 132.08 88.265) (size 1) (drill 0.5) (layers "F.Cu" "B.Cu") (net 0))
 (via (at 140.97 88.265) (size 1) (drill 0.5) (layers "F.Cu" "B.Cu") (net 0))
 (via (at 127.635 83.82) (size 1) (drill 0.5) (layers "F.Cu" "B.Cu") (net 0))
 (via (at 150.495 82.55) (size 1) (drill 0.5) (layers "F.Cu" "B.Cu") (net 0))
 (via (at 150.495 80.01) (size 1) (drill 0.5) (layers "F.Cu" "B.Cu") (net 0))
 (via (at 146.05 65.405) (size 1) (drill 0.5) (layers "F.Cu" "B.Cu") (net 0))
 (via (at 137.16 88.265) (size 1) (drill 0.5) (layers "F.Cu" "B.Cu") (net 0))
 (via (at 135.89 65.405) (size 1) (drill 0.5) (layers "F.Cu" "B.Cu") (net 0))
 (via (at 150.495 74.93) (size 1) (drill 0.5) (layers "F.Cu" "B.Cu") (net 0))
 (via (at 127.635 68.58) (size 1) (drill 0.5) (layers "F.Cu" "B.Cu") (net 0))
 (via (at 133.35 88.265) (size 1) (drill 0.5) (layers "F.Cu" "B.Cu") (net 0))
 (via (at 127.635 86.36) (size 1) (drill 0.5) (layers "F.Cu" "B.Cu") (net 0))
 (via (at 150.495 69.85) (size 1) (drill 0.5) (layers "F.Cu" "B.Cu") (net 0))
 (via (at 150.495 83.82) (size 1) (drill 0.5) (layers "F.Cu" "B.Cu") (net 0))
 (via (at 143.51 65.405) (size 1) (drill 0.5) (layers "F.Cu" "B.Cu") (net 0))
 (via (at 150.495 78.74) (size 1) (drill 0.5) (layers "F.Cu" "B.Cu") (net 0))
 (via (at 142.24 88.265) (size 1) (drill 0.5) (layers "F.Cu" "B.Cu") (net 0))
 (via (at 150.495 67.31) (size 1) (drill 0.5) (layers "F.Cu" "B.Cu") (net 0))
 (via (at 150.495 77.47) (size 1) (drill 0.5) (layers "F.Cu" "B.Cu") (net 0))
 (via (at 146.05 88.265) (size 1) (drill 0.5) (layers "F.Cu" "B.Cu") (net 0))
 (via (at 135.89 88.265) (size 1) (drill 0.5) (layers "F.Cu" "B.Cu") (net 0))
 (via (at 150.495 86.36) (size 1) (drill 0.5) (layers "F.Cu" "B.Cu") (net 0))
 (via (at 150.495 73.66) (size 1) (drill 0.5) (layers "F.Cu" "B.Cu") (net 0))
 (via (at 148.59 88.265) (size 1) (drill 0.5) (layers "F.Cu" "B.Cu") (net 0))
 (via (at 148.59 65.405) (size 1) (drill 0.5) (layers "F.Cu" "B.Cu") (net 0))
 (via (at 127.635 82.55) (size 1) (drill 0.5) (layers "F.Cu" "B.Cu") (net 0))
 (via (at 127.635 72.39) (size 1) (drill 0.5) (layers "F.Cu" "B.Cu") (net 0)))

